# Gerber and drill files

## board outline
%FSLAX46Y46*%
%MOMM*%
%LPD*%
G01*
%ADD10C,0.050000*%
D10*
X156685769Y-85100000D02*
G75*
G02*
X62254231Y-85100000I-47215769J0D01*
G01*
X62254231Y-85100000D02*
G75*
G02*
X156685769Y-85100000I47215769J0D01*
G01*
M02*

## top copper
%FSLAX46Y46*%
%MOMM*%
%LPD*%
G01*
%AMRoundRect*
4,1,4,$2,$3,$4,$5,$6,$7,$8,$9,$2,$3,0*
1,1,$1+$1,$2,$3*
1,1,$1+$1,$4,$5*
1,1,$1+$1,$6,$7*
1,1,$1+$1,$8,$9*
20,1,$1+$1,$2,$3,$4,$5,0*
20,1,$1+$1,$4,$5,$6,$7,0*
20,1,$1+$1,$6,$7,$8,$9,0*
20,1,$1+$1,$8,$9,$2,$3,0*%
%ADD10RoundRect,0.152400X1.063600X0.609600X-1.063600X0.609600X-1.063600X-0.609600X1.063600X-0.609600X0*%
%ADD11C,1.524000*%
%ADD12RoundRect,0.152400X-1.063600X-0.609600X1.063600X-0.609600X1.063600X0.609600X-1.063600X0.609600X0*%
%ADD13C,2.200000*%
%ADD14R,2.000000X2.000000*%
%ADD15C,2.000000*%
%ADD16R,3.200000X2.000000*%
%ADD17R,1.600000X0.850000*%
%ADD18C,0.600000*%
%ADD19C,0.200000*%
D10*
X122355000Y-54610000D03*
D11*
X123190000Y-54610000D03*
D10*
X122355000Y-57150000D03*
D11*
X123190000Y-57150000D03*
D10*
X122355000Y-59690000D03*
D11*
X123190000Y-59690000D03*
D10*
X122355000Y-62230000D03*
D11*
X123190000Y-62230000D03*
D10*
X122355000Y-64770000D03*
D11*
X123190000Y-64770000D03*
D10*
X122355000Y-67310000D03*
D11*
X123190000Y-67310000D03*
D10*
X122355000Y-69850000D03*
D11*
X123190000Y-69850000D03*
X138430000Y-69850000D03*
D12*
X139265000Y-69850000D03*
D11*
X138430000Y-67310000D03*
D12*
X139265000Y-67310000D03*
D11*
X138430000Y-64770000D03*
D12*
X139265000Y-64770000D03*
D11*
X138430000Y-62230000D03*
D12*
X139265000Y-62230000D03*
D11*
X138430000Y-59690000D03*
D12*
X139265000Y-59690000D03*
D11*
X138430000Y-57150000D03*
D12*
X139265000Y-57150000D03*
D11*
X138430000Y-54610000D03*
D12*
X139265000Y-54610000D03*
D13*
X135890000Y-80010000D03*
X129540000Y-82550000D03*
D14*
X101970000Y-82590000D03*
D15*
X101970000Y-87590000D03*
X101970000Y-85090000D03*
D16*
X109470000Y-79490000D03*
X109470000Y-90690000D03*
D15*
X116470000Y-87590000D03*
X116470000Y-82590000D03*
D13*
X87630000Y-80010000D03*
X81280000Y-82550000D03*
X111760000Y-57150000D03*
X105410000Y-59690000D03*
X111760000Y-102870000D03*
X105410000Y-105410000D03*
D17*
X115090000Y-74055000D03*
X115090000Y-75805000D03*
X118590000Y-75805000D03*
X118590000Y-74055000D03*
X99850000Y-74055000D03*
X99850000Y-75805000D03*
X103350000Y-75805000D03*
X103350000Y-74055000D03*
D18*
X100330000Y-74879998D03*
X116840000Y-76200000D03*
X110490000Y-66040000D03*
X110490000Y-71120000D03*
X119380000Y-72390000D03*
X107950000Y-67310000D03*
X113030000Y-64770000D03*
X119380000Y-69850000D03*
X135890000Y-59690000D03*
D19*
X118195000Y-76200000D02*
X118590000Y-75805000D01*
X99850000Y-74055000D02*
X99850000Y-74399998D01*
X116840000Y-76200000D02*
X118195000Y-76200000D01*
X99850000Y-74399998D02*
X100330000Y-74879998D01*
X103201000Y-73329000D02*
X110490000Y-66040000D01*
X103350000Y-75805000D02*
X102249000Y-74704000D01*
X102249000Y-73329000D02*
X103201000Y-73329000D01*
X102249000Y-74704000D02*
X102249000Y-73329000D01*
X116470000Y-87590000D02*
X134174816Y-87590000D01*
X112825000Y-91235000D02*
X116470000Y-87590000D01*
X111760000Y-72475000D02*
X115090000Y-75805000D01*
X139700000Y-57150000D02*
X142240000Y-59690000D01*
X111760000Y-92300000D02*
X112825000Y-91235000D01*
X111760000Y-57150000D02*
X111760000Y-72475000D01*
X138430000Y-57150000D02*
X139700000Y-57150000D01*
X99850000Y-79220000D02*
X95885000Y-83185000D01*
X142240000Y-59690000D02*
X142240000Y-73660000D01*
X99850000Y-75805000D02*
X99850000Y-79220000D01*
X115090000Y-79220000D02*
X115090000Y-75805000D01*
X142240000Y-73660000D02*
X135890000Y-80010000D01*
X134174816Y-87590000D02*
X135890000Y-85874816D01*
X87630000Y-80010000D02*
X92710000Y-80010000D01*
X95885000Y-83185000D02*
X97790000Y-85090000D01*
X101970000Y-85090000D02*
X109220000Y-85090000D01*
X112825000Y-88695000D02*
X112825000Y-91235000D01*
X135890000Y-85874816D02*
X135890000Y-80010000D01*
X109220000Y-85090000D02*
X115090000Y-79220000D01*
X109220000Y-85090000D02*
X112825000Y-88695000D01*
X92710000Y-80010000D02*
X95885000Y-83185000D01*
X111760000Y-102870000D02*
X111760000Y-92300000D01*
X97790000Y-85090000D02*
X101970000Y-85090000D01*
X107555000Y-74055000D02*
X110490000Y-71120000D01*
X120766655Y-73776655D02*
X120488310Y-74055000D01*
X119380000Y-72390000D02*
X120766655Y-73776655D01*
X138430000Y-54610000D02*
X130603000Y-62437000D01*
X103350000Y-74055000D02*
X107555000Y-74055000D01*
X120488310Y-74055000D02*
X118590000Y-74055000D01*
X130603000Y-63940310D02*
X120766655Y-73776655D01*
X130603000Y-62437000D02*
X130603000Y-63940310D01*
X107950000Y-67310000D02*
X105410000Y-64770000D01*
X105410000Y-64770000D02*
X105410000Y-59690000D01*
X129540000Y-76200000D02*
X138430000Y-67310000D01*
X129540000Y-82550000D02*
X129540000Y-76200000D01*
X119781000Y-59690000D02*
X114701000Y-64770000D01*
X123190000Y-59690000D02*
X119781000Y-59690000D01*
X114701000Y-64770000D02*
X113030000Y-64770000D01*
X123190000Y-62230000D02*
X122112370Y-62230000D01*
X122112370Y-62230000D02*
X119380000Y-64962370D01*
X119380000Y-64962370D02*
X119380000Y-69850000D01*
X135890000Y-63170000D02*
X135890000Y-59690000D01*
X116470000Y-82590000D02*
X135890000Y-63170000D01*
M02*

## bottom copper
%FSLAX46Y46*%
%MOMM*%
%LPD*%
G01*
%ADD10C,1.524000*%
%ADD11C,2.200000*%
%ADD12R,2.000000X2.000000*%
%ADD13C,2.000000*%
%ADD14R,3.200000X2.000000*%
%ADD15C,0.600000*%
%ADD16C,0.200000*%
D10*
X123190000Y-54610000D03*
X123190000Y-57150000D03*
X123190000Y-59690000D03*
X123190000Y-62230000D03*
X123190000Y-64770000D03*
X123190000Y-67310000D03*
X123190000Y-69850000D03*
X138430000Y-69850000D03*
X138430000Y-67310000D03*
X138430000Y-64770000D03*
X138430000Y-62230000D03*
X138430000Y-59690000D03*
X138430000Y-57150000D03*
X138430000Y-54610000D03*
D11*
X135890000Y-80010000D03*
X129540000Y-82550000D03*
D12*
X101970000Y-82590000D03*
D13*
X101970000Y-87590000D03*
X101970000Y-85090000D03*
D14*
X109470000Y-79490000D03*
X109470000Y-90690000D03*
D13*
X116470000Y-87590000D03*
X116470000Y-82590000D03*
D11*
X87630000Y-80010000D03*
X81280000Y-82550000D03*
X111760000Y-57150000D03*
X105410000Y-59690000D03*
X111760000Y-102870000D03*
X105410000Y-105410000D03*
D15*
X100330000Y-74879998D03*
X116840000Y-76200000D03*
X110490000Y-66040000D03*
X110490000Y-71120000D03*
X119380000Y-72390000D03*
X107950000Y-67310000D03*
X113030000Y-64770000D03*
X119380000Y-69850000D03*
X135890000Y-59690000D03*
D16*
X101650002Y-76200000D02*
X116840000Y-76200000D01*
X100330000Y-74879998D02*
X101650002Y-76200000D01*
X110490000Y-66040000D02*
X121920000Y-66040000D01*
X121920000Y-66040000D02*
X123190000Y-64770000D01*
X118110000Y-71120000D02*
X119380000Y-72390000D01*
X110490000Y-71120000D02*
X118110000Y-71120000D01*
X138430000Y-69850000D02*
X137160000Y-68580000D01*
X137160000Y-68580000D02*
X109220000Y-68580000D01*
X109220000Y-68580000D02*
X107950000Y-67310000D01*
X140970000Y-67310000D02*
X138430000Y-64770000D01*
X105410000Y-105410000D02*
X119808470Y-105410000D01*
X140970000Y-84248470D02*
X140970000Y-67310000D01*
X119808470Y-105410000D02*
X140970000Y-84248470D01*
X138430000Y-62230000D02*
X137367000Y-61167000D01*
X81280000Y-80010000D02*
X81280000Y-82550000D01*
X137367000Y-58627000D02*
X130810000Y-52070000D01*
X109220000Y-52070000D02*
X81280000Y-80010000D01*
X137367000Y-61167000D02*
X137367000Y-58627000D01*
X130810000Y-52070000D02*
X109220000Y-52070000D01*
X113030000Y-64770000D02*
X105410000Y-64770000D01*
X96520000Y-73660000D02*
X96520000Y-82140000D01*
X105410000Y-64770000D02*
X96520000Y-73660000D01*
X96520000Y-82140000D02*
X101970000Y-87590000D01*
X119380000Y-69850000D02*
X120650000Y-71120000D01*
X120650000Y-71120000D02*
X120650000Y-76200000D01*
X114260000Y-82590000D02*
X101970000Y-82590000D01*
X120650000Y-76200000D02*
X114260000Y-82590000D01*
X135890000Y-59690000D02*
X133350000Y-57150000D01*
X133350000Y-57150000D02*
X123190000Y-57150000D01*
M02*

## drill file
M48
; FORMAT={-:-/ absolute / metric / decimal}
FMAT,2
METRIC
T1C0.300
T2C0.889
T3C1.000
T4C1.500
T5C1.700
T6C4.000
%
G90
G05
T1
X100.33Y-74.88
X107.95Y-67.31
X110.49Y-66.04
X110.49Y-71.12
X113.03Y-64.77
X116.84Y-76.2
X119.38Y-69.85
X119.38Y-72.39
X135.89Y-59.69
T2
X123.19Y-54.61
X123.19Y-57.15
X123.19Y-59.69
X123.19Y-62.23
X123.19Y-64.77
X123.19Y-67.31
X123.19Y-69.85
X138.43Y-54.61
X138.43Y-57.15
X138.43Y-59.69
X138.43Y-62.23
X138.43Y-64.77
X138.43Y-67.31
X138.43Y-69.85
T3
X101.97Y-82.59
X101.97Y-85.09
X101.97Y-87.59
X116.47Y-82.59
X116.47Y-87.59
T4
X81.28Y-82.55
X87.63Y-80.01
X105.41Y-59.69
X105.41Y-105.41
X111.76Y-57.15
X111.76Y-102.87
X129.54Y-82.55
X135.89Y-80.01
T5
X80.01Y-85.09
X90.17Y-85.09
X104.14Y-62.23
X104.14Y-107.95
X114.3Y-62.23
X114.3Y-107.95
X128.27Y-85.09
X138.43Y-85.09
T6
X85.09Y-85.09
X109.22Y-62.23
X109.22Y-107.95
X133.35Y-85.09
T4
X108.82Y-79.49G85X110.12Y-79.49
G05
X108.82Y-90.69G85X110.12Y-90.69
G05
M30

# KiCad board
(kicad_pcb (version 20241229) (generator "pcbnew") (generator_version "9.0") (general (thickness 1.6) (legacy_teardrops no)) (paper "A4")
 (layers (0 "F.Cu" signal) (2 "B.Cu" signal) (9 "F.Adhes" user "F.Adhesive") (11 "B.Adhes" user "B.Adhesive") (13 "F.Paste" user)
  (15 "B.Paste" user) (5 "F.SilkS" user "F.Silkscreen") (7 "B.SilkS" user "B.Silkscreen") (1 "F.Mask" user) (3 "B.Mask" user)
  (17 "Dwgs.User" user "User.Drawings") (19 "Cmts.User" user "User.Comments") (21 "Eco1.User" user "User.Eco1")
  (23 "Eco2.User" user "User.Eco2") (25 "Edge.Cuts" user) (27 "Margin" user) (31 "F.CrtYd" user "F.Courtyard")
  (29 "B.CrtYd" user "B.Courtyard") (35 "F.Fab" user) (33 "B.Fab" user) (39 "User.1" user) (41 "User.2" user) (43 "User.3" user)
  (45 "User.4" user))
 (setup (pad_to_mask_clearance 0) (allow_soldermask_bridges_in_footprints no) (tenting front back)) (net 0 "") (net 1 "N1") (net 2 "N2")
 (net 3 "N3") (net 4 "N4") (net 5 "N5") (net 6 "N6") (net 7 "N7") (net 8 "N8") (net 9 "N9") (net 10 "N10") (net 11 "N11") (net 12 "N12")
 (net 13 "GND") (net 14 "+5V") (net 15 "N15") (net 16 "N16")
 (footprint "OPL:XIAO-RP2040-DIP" (layer "F.Cu") (at 130.81 62.23)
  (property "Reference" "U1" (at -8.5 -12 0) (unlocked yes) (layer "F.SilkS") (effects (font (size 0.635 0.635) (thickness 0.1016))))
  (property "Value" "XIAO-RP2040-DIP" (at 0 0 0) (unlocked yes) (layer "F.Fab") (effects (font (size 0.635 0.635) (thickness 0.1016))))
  (pad "1" smd roundrect (at -8.455 -7.62 180) (size 2.432 1.524) (layers "F.Cu" "F.Mask") (roundrect_rratio 0.1) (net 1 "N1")
   (thermal_bridge_angle 45))
  (pad "1" thru_hole circle (at -7.62 -7.62 180) (size 1.524 1.524) (drill 0.889) (layers "*.Cu" "*.Mask") (remove_unused_layers no)
   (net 1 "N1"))
  (pad "2" smd roundrect (at -8.455 -5.08 180) (size 2.432 1.524) (layers "F.Cu" "F.Mask") (roundrect_rratio 0.1) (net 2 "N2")
   (thermal_bridge_angle 45))
  (pad "2" thru_hole circle (at -7.62 -5.08 180) (size 1.524 1.524) (drill 0.889) (layers "*.Cu" "*.Mask") (remove_unused_layers no)
   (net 2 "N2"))
  (pad "3" smd roundrect (at -8.455 -2.54 180) (size 2.432 1.524) (layers "F.Cu" "F.Mask") (roundrect_rratio 0.1) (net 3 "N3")
   (thermal_bridge_angle 45))
  (pad "3" thru_hole circle (at -7.62 -2.54 180) (size 1.524 1.524) (drill 0.889) (layers "*.Cu" "*.Mask") (remove_unused_layers no)
   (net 3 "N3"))
  (pad "4" smd roundrect (at -8.455 0 180) (size 2.432 1.524) (layers "F.Cu" "F.Mask") (roundrect_rratio 0.1) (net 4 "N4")
   (thermal_bridge_angle 45))
  (pad "4" thru_hole circle (at -7.62 0 180) (size 1.524 1.524) (drill 0.889) (layers "*.Cu" "*.Mask") (remove_unused_layers no)
   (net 4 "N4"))
  (pad "5" smd roundrect (at -8.455 2.54 180) (size 2.432 1.524) (layers "F.Cu" "F.Mask") (roundrect_rratio 0.1) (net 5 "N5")
   (thermal_bridge_angle 45))
  (pad "5" thru_hole circle (at -7.62 2.54 180) (size 1.524 1.524) (drill 0.889) (layers "*.Cu" "*.Mask") (remove_unused_layers no)
   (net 5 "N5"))
  (pad "6" smd roundrect (at -8.455 5.08 180) (size 2.432 1.524) (layers "F.Cu" "F.Mask") (roundrect_rratio 0.1) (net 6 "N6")
   (thermal_bridge_angle 45))
  (pad "6" thru_hole circle (at -7.62 5.08 180) (size 1.524 1.524) (drill 0.889) (layers "*.Cu" "*.Mask") (remove_unused_layers no)
   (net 6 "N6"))
  (pad "7" smd roundrect (at -8.455 7.62 180) (size 2.432 1.524) (layers "F.Cu" "F.Mask") (roundrect_rratio 0.1) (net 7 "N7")
   (thermal_bridge_angle 45))
  (pad "7" thru_hole circle (at -7.62 7.62 180) (size 1.524 1.524) (drill 0.889) (layers "*.Cu" "*.Mask") (remove_unused_layers no)
   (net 7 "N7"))
  (pad "8" thru_hole circle (at 7.62 7.62) (size 1.524 1.524) (drill 0.889) (layers "*.Cu" "*.Mask") (remove_unused_layers no) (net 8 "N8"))
  (pad "8" smd roundrect (at 8.455 7.62) (size 2.432 1.524) (layers "F.Cu" "F.Mask") (roundrect_rratio 0.1) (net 8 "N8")
   (thermal_bridge_angle 45))
  (pad "9" thru_hole circle (at 7.62 5.08) (size 1.524 1.524) (drill 0.889) (layers "*.Cu" "*.Mask") (remove_unused_layers no) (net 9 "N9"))
  (pad "9" smd roundrect (at 8.455 5.08) (size 2.432 1.524) (layers "F.Cu" "F.Mask") (roundrect_rratio 0.1) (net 9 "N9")
   (thermal_bridge_angle 45))
  (pad "10" thru_hole circle (at 7.62 2.54) (size 1.524 1.524) (drill 0.889) (layers "*.Cu" "*.Mask") (remove_unused_layers no)
   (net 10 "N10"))
  (pad "10" smd roundrect (at 8.455 2.54) (size 2.432 1.524) (layers "F.Cu" "F.Mask") (roundrect_rratio 0.1) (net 10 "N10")
   (thermal_bridge_angle 45))
  (pad "11" thru_hole circle (at 7.62 0) (size 1.524 1.524) (drill 0.889) (layers "*.Cu" "*.Mask") (remove_unused_layers no) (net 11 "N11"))
  (pad "11" smd roundrect (at 8.455 0) (size 2.432 1.524) (layers "F.Cu" "F.Mask") (roundrect_rratio 0.1) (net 11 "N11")
   (thermal_bridge_angle 45))
  (pad "12" thru_hole circle (at 7.62 -2.54) (size 1.524 1.524) (drill 0.889) (layers "*.Cu" "*.Mask") (remove_unused_layers no)
   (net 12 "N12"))
  (pad "12" smd roundrect (at 8.455 -2.54) (size 2.432 1.524) (layers "F.Cu" "F.Mask") (roundrect_rratio 0.1) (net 12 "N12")
   (thermal_bridge_angle 45))
  (pad "13" thru_hole circle (at 7.62 -5.08) (size 1.524 1.524) (drill 0.889) (layers "*.Cu" "*.Mask") (remove_unused_layers no)
   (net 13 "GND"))
  (pad "13" smd roundrect (at 8.455 -5.08) (size 2.432 1.524) (layers "F.Cu" "F.Mask") (roundrect_rratio 0.1) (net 13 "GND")
   (thermal_bridge_angle 45))
  (pad "14" thru_hole circle (at 7.62 -7.62) (size 1.524 1.524) (drill 0.889) (layers "*.Cu" "*.Mask") (remove_unused_layers no)
   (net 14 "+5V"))
  (pad "14" smd roundrect (at 8.455 -7.62) (size 2.432 1.524) (layers "F.Cu" "F.Mask") (roundrect_rratio 0.1) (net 14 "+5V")
   (thermal_bridge_angle 45)))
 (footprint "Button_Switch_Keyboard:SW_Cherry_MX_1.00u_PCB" (layer "F.Cu") (at 135.89 80.01)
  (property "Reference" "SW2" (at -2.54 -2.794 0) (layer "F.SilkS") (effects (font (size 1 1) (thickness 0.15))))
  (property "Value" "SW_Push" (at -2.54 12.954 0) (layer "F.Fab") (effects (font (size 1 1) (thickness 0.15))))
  (pad "" np_thru_hole circle (at -7.62 5.08) (size 1.7 1.7) (drill 1.7) (layers "*.Cu" "*.Mask"))
  (pad "" np_thru_hole circle (at -2.54 5.08) (size 4 4) (drill 4) (layers "*.Cu" "*.Mask"))
  (pad "" np_thru_hole circle (at 2.54 5.08) (size 1.7 1.7) (drill 1.7) (layers "*.Cu" "*.Mask"))
  (pad "1" thru_hole circle (at 0 0) (size 2.2 2.2) (drill 1.5) (layers "*.Cu" "*.Mask") (remove_unused_layers no) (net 13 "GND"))
  (pad "2" thru_hole circle (at -6.35 2.54) (size 2.2 2.2) (drill 1.5) (layers "*.Cu" "*.Mask") (remove_unused_layers no) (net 9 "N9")))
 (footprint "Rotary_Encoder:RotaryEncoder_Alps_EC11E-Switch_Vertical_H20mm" (layer "F.Cu") (at 101.97 82.59)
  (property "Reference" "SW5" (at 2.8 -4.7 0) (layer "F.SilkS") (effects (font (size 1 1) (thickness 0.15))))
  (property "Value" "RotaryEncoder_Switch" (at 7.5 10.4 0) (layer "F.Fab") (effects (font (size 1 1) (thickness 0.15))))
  (pad "A" thru_hole rect (at 0 0) (size 2 2) (drill 1) (layers "*.Cu" "*.Mask") (remove_unused_layers no) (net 4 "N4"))
  (pad "B" thru_hole circle (at 0 5) (size 2 2) (drill 1) (layers "*.Cu" "*.Mask") (remove_unused_layers no) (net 3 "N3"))
  (pad "C" thru_hole circle (at 0 2.5) (size 2 2) (drill 1) (layers "*.Cu" "*.Mask") (remove_unused_layers no) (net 13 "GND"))
  (pad "MP" thru_hole rect (at 7.5 -3.1) (size 3.2 2) (drill oval 2.8 1.5) (layers "*.Cu" "*.Mask") (remove_unused_layers no))
  (pad "MP" thru_hole rect (at 7.5 8.1) (size 3.2 2) (drill oval 2.8 1.5) (layers "*.Cu" "*.Mask") (remove_unused_layers no))
  (pad "S1" thru_hole circle (at 14.5 5) (size 2 2) (drill 1) (layers "*.Cu" "*.Mask") (remove_unused_layers no) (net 13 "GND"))
  (pad "S2" thru_hole circle (at 14.5 0) (size 2 2) (drill 1) (layers "*.Cu" "*.Mask") (remove_unused_layers no) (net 2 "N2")))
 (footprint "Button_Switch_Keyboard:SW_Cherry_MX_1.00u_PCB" (layer "F.Cu") (at 87.63 80.01)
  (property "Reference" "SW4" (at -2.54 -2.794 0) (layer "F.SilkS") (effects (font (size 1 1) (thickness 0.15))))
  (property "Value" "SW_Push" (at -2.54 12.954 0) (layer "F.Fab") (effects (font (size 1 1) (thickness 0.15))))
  (pad "" np_thru_hole circle (at -7.62 5.08) (size 1.7 1.7) (drill 1.7) (layers "*.Cu" "*.Mask"))
  (pad "" np_thru_hole circle (at -2.54 5.08) (size 4 4) (drill 4) (layers "*.Cu" "*.Mask"))
  (pad "" np_thru_hole circle (at 2.54 5.08) (size 1.7 1.7) (drill 1.7) (layers "*.Cu" "*.Mask"))
  (pad "1" thru_hole circle (at 0 0) (size 2.2 2.2) (drill 1.5) (layers "*.Cu" "*.Mask") (remove_unused_layers no) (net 13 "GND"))
  (pad "2" thru_hole circle (at -6.35 2.54) (size 2.2 2.2) (drill 1.5) (layers "*.Cu" "*.Mask") (remove_unused_layers no) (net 11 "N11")))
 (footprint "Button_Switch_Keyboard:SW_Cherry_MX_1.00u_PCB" (layer "F.Cu") (at 111.76 57.15)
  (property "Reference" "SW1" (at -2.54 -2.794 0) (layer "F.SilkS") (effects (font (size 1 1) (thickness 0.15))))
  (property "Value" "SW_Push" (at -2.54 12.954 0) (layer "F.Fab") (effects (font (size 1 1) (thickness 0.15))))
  (pad "" np_thru_hole circle (at -7.62 5.08) (size 1.7 1.7) (drill 1.7) (layers "*.Cu" "*.Mask"))
  (pad "" np_thru_hole circle (at -2.54 5.08) (size 4 4) (drill 4) (layers "*.Cu" "*.Mask"))
  (pad "" np_thru_hole circle (at 2.54 5.08) (size 1.7 1.7) (drill 1.7) (layers "*.Cu" "*.Mask"))
  (pad "1" thru_hole circle (at 0 0) (size 2.2 2.2) (drill 1.5) (layers "*.Cu" "*.Mask") (remove_unused_layers no) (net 13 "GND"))
  (pad "2" thru_hole circle (at -6.35 2.54) (size 2.2 2.2) (drill 1.5) (layers "*.Cu" "*.Mask") (remove_unused_layers no) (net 8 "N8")))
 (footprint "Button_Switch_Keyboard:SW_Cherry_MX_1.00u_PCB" (layer "F.Cu") (at 111.76 102.87)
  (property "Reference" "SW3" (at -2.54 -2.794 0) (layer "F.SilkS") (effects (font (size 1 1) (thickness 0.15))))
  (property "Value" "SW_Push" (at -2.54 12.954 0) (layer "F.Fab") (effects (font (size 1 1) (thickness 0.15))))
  (pad "" np_thru_hole circle (at -7.62 5.08) (size 1.7 1.7) (drill 1.7) (layers "*.Cu" "*.Mask"))
  (pad "" np_thru_hole circle (at -2.54 5.08) (size 4 4) (drill 4) (layers "*.Cu" "*.Mask"))
  (pad "" np_thru_hole circle (at 2.54 5.08) (size 1.7 1.7) (drill 1.7) (layers "*.Cu" "*.Mask"))
  (pad "1" thru_hole circle (at 0 0) (size 2.2 2.2) (drill 1.5) (layers "*.Cu" "*.Mask") (remove_unused_layers no) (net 13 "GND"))
  (pad "2" thru_hole circle (at -6.35 2.54) (size 2.2 2.2) (drill 1.5) (layers "*.Cu" "*.Mask") (remove_unused_layers no) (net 10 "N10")))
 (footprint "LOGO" (layer "F.Cu") (at 83.98 62.84)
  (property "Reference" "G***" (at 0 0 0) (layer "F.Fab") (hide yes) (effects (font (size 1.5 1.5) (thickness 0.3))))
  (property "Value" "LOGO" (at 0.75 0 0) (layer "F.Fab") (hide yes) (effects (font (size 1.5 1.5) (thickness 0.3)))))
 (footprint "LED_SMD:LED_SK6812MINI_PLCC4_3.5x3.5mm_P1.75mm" (layer "F.Cu") (at 116.84 74.93)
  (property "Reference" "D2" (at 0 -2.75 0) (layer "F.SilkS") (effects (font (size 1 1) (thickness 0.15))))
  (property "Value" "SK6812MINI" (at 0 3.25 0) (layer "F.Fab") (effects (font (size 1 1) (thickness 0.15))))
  (pad "1" smd rect (at -1.75 -0.875) (size 1.6 0.85) (layers "F.Cu" "F.Mask" "F.Paste") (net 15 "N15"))
  (pad "2" smd rect (at -1.75 0.875) (size 1.6 0.85) (layers "F.Cu" "F.Mask" "F.Paste") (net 13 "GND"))
  (pad "3" smd rect (at 1.75 0.875) (size 1.6 0.85) (layers "F.Cu" "F.Mask" "F.Paste") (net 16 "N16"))
  (pad "4" smd rect (at 1.75 -0.875) (size 1.6 0.85) (layers "F.Cu" "F.Mask" "F.Paste") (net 14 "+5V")))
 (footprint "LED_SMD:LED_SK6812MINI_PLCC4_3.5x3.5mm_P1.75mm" (layer "F.Cu") (at 101.6 74.93)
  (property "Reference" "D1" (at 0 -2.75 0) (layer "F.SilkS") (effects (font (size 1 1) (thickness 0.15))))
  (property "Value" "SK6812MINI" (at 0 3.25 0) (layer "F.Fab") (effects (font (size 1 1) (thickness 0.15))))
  (pad "1" smd rect (at -1.75 -0.875) (size 1.6 0.85) (layers "F.Cu" "F.Mask" "F.Paste") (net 16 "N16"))
  (pad "2" smd rect (at -1.75 0.875) (size 1.6 0.85) (layers "F.Cu" "F.Mask" "F.Paste") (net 13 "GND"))
  (pad "3" smd rect (at 1.75 0.875) (size 1.6 0.85) (layers "F.Cu" "F.Mask" "F.Paste") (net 5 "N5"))
  (pad "4" smd rect (at 1.75 -0.875) (size 1.6 0.85) (layers "F.Cu" "F.Mask" "F.Paste") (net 14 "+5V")))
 (gr_circle (center 109.47 85.1) (end 129.45 127.88) (stroke (width 0.05) (type default)) (fill no) (layer "Edge.Cuts"))
 (segment (start 118.195 76.2) (end 118.59 75.805) (width 0.2) (layer "F.Cu") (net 16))
 (segment (start 99.85 74.055) (end 99.85 74.399998) (width 0.2) (layer "F.Cu") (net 16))
 (segment (start 116.84 76.2) (end 118.195 76.2) (width 0.2) (layer "F.Cu") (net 16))
 (segment (start 99.85 74.399998) (end 100.33 74.879998) (width 0.2) (layer "F.Cu") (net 16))
 (via (at 100.33 74.879998) (size 0.6) (drill 0.3) (layers "F.Cu" "B.Cu") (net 16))
 (via (at 116.84 76.2) (size 0.6) (drill 0.3) (layers "F.Cu" "B.Cu") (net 16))
 (segment (start 101.650002 76.2) (end 116.84 76.2) (width 0.2) (layer "B.Cu") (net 16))
 (segment (start 100.33 74.879998) (end 101.650002 76.2) (width 0.2) (layer "B.Cu") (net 16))
 (segment (start 103.201 73.329) (end 110.49 66.04) (width 0.2) (layer "F.Cu") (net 5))
 (segment (start 103.35 75.805) (end 102.249 74.704) (width 0.2) (layer "F.Cu") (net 5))
 (segment (start 102.249 73.329) (end 103.201 73.329) (width 0.2) (layer "F.Cu") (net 5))
 (segment (start 102.249 74.704) (end 102.249 73.329) (width 0.2) (layer "F.Cu") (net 5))
 (via (at 110.49 66.04) (size 0.6) (drill 0.3) (layers "F.Cu" "B.Cu") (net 5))
 (segment (start 110.49 66.04) (end 121.92 66.04) (width 0.2) (layer "B.Cu") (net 5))
 (segment (start 121.92 66.04) (end 123.19 64.77) (width 0.2) (layer "B.Cu") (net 5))
 (segment (start 116.47 87.59) (end 134.174816 87.59) (width 0.2) (layer "F.Cu") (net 13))
 (segment (start 112.825 91.235) (end 116.47 87.59) (width 0.2) (layer "F.Cu") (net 13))
 (segment (start 111.76 72.475) (end 115.09 75.805) (width 0.2) (layer "F.Cu") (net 13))
 (segment (start 139.7 57.15) (end 142.24 59.69) (width 0.2) (layer "F.Cu") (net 13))
 (segment (start 111.76 92.3) (end 112.825 91.235) (width 0.2) (layer "F.Cu") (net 13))
 (segment (start 111.76 57.15) (end 111.76 72.475) (width 0.2) (layer "F.Cu") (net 13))
 (segment (start 138.43 57.15) (end 139.7 57.15) (width 0.2) (layer "F.Cu") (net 13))
 (segment (start 99.85 79.22) (end 95.885 83.185) (width 0.2) (layer "F.Cu") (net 13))
 (segment (start 142.24 59.69) (end 142.24 73.66) (width 0.2) (layer "F.Cu") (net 13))
 (segment (start 99.85 75.805) (end 99.85 79.22) (width 0.2) (layer "F.Cu") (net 13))
 (segment (start 115.09 79.22) (end 115.09 75.805) (width 0.2) (layer "F.Cu") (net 13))
 (segment (start 142.24 73.66) (end 135.89 80.01) (width 0.2) (layer "F.Cu") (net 13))
 (segment (start 134.174816 87.59) (end 135.89 85.874816) (width 0.2) (layer "F.Cu") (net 13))
 (segment (start 87.63 80.01) (end 92.71 80.01) (width 0.2) (layer "F.Cu") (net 13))
 (segment (start 95.885 83.185) (end 97.79 85.09) (width 0.2) (layer "F.Cu") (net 13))
 (segment (start 101.97 85.09) (end 109.22 85.09) (width 0.2) (layer "F.Cu") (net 13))
 (segment (start 112.825 88.695) (end 112.825 91.235) (width 0.2) (layer "F.Cu") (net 13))
 (segment (start 135.89 85.874816) (end 135.89 80.01) (width 0.2) (layer "F.Cu") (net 13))
 (segment (start 109.22 85.09) (end 115.09 79.22) (width 0.2) (layer "F.Cu") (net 13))
 (segment (start 109.22 85.09) (end 112.825 88.695) (width 0.2) (layer "F.Cu") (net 13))
 (segment (start 92.71 80.01) (end 95.885 83.185) (width 0.2) (layer "F.Cu") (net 13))
 (segment (start 111.76 102.87) (end 111.76 92.3) (width 0.2) (layer "F.Cu") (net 13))
 (segment (start 97.79 85.09) (end 101.97 85.09) (width 0.2) (layer "F.Cu") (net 13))
 (segment (start 107.555 74.055) (end 110.49 71.12) (width 0.2) (layer "F.Cu") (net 14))
 (segment (start 120.766655 73.776655) (end 120.48831 74.055) (width 0.2) (layer "F.Cu") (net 14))
 (segment (start 119.38 72.39) (end 120.766655 73.776655) (width 0.2) (layer "F.Cu") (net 14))
 (segment (start 138.43 54.61) (end 130.603 62.437) (width 0.2) (layer "F.Cu") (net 14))
 (segment (start 103.35 74.055) (end 107.555 74.055) (width 0.2) (layer "F.Cu") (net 14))
 (segment (start 120.48831 74.055) (end 118.59 74.055) (width 0.2) (layer "F.Cu") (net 14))
 (segment (start 130.603 63.94031) (end 120.766655 73.776655) (width 0.2) (layer "F.Cu") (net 14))
 (segment (start 130.603 62.437) (end 130.603 63.94031) (width 0.2) (layer "F.Cu") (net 14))
 (via (at 110.49 71.12) (size 0.6) (drill 0.3) (layers "F.Cu" "B.Cu") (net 14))
 (via (at 119.38 72.39) (size 0.6) (drill 0.3) (layers "F.Cu" "B.Cu") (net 14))
 (segment (start 118.11 71.12) (end 119.38 72.39) (width 0.2) (layer "B.Cu") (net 14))
 (segment (start 110.49 71.12) (end 118.11 71.12) (width 0.2) (layer "B.Cu") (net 14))
 (segment (start 107.95 67.31) (end 105.41 64.77) (width 0.2) (layer "F.Cu") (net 8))
 (segment (start 105.41 64.77) (end 105.41 59.69) (width 0.2) (layer "F.Cu") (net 8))
 (via (at 107.95 67.31) (size 0.6) (drill 0.3) (layers "F.Cu" "B.Cu") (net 8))
 (segment (start 138.43 69.85) (end 137.16 68.58) (width 0.2) (layer "B.Cu") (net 8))
 (segment (start 137.16 68.58) (end 109.22 68.58) (width 0.2) (layer "B.Cu") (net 8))
 (segment (start 109.22 68.58) (end 107.95 67.31) (width 0.2) (layer "B.Cu") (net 8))
 (segment (start 129.54 76.2) (end 138.43 67.31) (width 0.2) (layer "F.Cu") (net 9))
 (segment (start 129.54 82.55) (end 129.54 76.2) (width 0.2) (layer "F.Cu") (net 9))
 (segment (start 140.97 67.31) (end 138.43 64.77) (width 0.2) (layer "B.Cu") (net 10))
 (segment (start 105.41 105.41) (end 119.80847 105.41) (width 0.2) (layer "B.Cu") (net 10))
 (segment (start 140.97 84.24847) (end 140.97 67.31) (width 0.2) (layer "B.Cu") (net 10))
 (segment (start 119.80847 105.41) (end 140.97 84.24847) (width 0.2) (layer "B.Cu") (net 10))
 (segment (start 138.43 62.23) (end 137.367 61.167) (width 0.2) (layer "B.Cu") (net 11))
 (segment (start 81.28 80.01) (end 81.28 82.55) (width 0.2) (layer "B.Cu") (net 11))
 (segment (start 137.367 58.627) (end 130.81 52.07) (width 0.2) (layer "B.Cu") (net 11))
 (segment (start 109.22 52.07) (end 81.28 80.01) (width 0.2) (layer "B.Cu") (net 11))
 (segment (start 137.367 61.167) (end 137.367 58.627) (width 0.2) (layer "B.Cu") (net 11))
 (segment (start 130.81 52.07) (end 109.22 52.07) (width 0.2) (layer "B.Cu") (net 11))
 (segment (start 119.781 59.69) (end 114.701 64.77) (width 0.2) (layer "F.Cu") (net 3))
 (segment (start 123.19 59.69) (end 119.781 59.69) (width 0.2) (layer "F.Cu") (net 3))
 (segment (start 114.701 64.77) (end 113.03 64.77) (width 0.2) (layer "F.Cu") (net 3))
 (via (at 113.03 64.77) (size 0.6) (drill 0.3) (layers "F.Cu" "B.Cu") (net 3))
 (segment (start 113.03 64.77) (end 105.41 64.77) (width 0.2) (layer "B.Cu") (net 3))
 (segment (start 96.52 73.66) (end 96.52 82.14) (width 0.2) (layer "B.Cu") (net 3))
 (segment (start 105.41 64.77) (end 96.52 73.66) (width 0.2) (layer "B.Cu") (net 3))
 (segment (start 96.52 82.14) (end 101.97 87.59) (width 0.2) (layer "B.Cu") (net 3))
 (segment (start 123.19 62.23) (end 122.11237 62.23) (width 0.2) (layer "F.Cu") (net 4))
 (segment (start 122.11237 62.23) (end 119.38 64.96237) (width 0.2) (layer "F.Cu") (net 4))
 (segment (start 119.38 64.96237) (end 119.38 69.85) (width 0.2) (layer "F.Cu") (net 4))
 (via (at 119.38 69.85) (size 0.6) (drill 0.3) (layers "F.Cu" "B.Cu") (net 4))
 (segment (start 119.38 69.85) (end 120.65 71.12) (width 0.2) (layer "B.Cu") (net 4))
 (segment (start 120.65 71.12) (end 120.65 76.2) (width 0.2) (layer "B.Cu") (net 4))
 (segment (start 114.26 82.59) (end 101.97 82.59) (width 0.2) (layer "B.Cu") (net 4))
 (segment (start 120.65 76.2) (end 114.26 82.59) (width 0.2) (layer "B.Cu") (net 4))
 (segment (start 135.89 63.17) (end 135.89 59.69) (width 0.2) (layer "F.Cu") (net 2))
 (segment (start 116.47 82.59) (end 135.89 63.17) (width 0.2) (layer "F.Cu") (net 2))
 (via (at 135.89 59.69) (size 0.6) (drill 0.3) (layers "F.Cu" "B.Cu") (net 2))
 (segment (start 135.89 59.69) (end 133.35 57.15) (width 0.2) (layer "B.Cu") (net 2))
 (segment (start 133.35 57.15) (end 123.19 57.15) (width 0.2) (layer "B.Cu") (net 2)))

